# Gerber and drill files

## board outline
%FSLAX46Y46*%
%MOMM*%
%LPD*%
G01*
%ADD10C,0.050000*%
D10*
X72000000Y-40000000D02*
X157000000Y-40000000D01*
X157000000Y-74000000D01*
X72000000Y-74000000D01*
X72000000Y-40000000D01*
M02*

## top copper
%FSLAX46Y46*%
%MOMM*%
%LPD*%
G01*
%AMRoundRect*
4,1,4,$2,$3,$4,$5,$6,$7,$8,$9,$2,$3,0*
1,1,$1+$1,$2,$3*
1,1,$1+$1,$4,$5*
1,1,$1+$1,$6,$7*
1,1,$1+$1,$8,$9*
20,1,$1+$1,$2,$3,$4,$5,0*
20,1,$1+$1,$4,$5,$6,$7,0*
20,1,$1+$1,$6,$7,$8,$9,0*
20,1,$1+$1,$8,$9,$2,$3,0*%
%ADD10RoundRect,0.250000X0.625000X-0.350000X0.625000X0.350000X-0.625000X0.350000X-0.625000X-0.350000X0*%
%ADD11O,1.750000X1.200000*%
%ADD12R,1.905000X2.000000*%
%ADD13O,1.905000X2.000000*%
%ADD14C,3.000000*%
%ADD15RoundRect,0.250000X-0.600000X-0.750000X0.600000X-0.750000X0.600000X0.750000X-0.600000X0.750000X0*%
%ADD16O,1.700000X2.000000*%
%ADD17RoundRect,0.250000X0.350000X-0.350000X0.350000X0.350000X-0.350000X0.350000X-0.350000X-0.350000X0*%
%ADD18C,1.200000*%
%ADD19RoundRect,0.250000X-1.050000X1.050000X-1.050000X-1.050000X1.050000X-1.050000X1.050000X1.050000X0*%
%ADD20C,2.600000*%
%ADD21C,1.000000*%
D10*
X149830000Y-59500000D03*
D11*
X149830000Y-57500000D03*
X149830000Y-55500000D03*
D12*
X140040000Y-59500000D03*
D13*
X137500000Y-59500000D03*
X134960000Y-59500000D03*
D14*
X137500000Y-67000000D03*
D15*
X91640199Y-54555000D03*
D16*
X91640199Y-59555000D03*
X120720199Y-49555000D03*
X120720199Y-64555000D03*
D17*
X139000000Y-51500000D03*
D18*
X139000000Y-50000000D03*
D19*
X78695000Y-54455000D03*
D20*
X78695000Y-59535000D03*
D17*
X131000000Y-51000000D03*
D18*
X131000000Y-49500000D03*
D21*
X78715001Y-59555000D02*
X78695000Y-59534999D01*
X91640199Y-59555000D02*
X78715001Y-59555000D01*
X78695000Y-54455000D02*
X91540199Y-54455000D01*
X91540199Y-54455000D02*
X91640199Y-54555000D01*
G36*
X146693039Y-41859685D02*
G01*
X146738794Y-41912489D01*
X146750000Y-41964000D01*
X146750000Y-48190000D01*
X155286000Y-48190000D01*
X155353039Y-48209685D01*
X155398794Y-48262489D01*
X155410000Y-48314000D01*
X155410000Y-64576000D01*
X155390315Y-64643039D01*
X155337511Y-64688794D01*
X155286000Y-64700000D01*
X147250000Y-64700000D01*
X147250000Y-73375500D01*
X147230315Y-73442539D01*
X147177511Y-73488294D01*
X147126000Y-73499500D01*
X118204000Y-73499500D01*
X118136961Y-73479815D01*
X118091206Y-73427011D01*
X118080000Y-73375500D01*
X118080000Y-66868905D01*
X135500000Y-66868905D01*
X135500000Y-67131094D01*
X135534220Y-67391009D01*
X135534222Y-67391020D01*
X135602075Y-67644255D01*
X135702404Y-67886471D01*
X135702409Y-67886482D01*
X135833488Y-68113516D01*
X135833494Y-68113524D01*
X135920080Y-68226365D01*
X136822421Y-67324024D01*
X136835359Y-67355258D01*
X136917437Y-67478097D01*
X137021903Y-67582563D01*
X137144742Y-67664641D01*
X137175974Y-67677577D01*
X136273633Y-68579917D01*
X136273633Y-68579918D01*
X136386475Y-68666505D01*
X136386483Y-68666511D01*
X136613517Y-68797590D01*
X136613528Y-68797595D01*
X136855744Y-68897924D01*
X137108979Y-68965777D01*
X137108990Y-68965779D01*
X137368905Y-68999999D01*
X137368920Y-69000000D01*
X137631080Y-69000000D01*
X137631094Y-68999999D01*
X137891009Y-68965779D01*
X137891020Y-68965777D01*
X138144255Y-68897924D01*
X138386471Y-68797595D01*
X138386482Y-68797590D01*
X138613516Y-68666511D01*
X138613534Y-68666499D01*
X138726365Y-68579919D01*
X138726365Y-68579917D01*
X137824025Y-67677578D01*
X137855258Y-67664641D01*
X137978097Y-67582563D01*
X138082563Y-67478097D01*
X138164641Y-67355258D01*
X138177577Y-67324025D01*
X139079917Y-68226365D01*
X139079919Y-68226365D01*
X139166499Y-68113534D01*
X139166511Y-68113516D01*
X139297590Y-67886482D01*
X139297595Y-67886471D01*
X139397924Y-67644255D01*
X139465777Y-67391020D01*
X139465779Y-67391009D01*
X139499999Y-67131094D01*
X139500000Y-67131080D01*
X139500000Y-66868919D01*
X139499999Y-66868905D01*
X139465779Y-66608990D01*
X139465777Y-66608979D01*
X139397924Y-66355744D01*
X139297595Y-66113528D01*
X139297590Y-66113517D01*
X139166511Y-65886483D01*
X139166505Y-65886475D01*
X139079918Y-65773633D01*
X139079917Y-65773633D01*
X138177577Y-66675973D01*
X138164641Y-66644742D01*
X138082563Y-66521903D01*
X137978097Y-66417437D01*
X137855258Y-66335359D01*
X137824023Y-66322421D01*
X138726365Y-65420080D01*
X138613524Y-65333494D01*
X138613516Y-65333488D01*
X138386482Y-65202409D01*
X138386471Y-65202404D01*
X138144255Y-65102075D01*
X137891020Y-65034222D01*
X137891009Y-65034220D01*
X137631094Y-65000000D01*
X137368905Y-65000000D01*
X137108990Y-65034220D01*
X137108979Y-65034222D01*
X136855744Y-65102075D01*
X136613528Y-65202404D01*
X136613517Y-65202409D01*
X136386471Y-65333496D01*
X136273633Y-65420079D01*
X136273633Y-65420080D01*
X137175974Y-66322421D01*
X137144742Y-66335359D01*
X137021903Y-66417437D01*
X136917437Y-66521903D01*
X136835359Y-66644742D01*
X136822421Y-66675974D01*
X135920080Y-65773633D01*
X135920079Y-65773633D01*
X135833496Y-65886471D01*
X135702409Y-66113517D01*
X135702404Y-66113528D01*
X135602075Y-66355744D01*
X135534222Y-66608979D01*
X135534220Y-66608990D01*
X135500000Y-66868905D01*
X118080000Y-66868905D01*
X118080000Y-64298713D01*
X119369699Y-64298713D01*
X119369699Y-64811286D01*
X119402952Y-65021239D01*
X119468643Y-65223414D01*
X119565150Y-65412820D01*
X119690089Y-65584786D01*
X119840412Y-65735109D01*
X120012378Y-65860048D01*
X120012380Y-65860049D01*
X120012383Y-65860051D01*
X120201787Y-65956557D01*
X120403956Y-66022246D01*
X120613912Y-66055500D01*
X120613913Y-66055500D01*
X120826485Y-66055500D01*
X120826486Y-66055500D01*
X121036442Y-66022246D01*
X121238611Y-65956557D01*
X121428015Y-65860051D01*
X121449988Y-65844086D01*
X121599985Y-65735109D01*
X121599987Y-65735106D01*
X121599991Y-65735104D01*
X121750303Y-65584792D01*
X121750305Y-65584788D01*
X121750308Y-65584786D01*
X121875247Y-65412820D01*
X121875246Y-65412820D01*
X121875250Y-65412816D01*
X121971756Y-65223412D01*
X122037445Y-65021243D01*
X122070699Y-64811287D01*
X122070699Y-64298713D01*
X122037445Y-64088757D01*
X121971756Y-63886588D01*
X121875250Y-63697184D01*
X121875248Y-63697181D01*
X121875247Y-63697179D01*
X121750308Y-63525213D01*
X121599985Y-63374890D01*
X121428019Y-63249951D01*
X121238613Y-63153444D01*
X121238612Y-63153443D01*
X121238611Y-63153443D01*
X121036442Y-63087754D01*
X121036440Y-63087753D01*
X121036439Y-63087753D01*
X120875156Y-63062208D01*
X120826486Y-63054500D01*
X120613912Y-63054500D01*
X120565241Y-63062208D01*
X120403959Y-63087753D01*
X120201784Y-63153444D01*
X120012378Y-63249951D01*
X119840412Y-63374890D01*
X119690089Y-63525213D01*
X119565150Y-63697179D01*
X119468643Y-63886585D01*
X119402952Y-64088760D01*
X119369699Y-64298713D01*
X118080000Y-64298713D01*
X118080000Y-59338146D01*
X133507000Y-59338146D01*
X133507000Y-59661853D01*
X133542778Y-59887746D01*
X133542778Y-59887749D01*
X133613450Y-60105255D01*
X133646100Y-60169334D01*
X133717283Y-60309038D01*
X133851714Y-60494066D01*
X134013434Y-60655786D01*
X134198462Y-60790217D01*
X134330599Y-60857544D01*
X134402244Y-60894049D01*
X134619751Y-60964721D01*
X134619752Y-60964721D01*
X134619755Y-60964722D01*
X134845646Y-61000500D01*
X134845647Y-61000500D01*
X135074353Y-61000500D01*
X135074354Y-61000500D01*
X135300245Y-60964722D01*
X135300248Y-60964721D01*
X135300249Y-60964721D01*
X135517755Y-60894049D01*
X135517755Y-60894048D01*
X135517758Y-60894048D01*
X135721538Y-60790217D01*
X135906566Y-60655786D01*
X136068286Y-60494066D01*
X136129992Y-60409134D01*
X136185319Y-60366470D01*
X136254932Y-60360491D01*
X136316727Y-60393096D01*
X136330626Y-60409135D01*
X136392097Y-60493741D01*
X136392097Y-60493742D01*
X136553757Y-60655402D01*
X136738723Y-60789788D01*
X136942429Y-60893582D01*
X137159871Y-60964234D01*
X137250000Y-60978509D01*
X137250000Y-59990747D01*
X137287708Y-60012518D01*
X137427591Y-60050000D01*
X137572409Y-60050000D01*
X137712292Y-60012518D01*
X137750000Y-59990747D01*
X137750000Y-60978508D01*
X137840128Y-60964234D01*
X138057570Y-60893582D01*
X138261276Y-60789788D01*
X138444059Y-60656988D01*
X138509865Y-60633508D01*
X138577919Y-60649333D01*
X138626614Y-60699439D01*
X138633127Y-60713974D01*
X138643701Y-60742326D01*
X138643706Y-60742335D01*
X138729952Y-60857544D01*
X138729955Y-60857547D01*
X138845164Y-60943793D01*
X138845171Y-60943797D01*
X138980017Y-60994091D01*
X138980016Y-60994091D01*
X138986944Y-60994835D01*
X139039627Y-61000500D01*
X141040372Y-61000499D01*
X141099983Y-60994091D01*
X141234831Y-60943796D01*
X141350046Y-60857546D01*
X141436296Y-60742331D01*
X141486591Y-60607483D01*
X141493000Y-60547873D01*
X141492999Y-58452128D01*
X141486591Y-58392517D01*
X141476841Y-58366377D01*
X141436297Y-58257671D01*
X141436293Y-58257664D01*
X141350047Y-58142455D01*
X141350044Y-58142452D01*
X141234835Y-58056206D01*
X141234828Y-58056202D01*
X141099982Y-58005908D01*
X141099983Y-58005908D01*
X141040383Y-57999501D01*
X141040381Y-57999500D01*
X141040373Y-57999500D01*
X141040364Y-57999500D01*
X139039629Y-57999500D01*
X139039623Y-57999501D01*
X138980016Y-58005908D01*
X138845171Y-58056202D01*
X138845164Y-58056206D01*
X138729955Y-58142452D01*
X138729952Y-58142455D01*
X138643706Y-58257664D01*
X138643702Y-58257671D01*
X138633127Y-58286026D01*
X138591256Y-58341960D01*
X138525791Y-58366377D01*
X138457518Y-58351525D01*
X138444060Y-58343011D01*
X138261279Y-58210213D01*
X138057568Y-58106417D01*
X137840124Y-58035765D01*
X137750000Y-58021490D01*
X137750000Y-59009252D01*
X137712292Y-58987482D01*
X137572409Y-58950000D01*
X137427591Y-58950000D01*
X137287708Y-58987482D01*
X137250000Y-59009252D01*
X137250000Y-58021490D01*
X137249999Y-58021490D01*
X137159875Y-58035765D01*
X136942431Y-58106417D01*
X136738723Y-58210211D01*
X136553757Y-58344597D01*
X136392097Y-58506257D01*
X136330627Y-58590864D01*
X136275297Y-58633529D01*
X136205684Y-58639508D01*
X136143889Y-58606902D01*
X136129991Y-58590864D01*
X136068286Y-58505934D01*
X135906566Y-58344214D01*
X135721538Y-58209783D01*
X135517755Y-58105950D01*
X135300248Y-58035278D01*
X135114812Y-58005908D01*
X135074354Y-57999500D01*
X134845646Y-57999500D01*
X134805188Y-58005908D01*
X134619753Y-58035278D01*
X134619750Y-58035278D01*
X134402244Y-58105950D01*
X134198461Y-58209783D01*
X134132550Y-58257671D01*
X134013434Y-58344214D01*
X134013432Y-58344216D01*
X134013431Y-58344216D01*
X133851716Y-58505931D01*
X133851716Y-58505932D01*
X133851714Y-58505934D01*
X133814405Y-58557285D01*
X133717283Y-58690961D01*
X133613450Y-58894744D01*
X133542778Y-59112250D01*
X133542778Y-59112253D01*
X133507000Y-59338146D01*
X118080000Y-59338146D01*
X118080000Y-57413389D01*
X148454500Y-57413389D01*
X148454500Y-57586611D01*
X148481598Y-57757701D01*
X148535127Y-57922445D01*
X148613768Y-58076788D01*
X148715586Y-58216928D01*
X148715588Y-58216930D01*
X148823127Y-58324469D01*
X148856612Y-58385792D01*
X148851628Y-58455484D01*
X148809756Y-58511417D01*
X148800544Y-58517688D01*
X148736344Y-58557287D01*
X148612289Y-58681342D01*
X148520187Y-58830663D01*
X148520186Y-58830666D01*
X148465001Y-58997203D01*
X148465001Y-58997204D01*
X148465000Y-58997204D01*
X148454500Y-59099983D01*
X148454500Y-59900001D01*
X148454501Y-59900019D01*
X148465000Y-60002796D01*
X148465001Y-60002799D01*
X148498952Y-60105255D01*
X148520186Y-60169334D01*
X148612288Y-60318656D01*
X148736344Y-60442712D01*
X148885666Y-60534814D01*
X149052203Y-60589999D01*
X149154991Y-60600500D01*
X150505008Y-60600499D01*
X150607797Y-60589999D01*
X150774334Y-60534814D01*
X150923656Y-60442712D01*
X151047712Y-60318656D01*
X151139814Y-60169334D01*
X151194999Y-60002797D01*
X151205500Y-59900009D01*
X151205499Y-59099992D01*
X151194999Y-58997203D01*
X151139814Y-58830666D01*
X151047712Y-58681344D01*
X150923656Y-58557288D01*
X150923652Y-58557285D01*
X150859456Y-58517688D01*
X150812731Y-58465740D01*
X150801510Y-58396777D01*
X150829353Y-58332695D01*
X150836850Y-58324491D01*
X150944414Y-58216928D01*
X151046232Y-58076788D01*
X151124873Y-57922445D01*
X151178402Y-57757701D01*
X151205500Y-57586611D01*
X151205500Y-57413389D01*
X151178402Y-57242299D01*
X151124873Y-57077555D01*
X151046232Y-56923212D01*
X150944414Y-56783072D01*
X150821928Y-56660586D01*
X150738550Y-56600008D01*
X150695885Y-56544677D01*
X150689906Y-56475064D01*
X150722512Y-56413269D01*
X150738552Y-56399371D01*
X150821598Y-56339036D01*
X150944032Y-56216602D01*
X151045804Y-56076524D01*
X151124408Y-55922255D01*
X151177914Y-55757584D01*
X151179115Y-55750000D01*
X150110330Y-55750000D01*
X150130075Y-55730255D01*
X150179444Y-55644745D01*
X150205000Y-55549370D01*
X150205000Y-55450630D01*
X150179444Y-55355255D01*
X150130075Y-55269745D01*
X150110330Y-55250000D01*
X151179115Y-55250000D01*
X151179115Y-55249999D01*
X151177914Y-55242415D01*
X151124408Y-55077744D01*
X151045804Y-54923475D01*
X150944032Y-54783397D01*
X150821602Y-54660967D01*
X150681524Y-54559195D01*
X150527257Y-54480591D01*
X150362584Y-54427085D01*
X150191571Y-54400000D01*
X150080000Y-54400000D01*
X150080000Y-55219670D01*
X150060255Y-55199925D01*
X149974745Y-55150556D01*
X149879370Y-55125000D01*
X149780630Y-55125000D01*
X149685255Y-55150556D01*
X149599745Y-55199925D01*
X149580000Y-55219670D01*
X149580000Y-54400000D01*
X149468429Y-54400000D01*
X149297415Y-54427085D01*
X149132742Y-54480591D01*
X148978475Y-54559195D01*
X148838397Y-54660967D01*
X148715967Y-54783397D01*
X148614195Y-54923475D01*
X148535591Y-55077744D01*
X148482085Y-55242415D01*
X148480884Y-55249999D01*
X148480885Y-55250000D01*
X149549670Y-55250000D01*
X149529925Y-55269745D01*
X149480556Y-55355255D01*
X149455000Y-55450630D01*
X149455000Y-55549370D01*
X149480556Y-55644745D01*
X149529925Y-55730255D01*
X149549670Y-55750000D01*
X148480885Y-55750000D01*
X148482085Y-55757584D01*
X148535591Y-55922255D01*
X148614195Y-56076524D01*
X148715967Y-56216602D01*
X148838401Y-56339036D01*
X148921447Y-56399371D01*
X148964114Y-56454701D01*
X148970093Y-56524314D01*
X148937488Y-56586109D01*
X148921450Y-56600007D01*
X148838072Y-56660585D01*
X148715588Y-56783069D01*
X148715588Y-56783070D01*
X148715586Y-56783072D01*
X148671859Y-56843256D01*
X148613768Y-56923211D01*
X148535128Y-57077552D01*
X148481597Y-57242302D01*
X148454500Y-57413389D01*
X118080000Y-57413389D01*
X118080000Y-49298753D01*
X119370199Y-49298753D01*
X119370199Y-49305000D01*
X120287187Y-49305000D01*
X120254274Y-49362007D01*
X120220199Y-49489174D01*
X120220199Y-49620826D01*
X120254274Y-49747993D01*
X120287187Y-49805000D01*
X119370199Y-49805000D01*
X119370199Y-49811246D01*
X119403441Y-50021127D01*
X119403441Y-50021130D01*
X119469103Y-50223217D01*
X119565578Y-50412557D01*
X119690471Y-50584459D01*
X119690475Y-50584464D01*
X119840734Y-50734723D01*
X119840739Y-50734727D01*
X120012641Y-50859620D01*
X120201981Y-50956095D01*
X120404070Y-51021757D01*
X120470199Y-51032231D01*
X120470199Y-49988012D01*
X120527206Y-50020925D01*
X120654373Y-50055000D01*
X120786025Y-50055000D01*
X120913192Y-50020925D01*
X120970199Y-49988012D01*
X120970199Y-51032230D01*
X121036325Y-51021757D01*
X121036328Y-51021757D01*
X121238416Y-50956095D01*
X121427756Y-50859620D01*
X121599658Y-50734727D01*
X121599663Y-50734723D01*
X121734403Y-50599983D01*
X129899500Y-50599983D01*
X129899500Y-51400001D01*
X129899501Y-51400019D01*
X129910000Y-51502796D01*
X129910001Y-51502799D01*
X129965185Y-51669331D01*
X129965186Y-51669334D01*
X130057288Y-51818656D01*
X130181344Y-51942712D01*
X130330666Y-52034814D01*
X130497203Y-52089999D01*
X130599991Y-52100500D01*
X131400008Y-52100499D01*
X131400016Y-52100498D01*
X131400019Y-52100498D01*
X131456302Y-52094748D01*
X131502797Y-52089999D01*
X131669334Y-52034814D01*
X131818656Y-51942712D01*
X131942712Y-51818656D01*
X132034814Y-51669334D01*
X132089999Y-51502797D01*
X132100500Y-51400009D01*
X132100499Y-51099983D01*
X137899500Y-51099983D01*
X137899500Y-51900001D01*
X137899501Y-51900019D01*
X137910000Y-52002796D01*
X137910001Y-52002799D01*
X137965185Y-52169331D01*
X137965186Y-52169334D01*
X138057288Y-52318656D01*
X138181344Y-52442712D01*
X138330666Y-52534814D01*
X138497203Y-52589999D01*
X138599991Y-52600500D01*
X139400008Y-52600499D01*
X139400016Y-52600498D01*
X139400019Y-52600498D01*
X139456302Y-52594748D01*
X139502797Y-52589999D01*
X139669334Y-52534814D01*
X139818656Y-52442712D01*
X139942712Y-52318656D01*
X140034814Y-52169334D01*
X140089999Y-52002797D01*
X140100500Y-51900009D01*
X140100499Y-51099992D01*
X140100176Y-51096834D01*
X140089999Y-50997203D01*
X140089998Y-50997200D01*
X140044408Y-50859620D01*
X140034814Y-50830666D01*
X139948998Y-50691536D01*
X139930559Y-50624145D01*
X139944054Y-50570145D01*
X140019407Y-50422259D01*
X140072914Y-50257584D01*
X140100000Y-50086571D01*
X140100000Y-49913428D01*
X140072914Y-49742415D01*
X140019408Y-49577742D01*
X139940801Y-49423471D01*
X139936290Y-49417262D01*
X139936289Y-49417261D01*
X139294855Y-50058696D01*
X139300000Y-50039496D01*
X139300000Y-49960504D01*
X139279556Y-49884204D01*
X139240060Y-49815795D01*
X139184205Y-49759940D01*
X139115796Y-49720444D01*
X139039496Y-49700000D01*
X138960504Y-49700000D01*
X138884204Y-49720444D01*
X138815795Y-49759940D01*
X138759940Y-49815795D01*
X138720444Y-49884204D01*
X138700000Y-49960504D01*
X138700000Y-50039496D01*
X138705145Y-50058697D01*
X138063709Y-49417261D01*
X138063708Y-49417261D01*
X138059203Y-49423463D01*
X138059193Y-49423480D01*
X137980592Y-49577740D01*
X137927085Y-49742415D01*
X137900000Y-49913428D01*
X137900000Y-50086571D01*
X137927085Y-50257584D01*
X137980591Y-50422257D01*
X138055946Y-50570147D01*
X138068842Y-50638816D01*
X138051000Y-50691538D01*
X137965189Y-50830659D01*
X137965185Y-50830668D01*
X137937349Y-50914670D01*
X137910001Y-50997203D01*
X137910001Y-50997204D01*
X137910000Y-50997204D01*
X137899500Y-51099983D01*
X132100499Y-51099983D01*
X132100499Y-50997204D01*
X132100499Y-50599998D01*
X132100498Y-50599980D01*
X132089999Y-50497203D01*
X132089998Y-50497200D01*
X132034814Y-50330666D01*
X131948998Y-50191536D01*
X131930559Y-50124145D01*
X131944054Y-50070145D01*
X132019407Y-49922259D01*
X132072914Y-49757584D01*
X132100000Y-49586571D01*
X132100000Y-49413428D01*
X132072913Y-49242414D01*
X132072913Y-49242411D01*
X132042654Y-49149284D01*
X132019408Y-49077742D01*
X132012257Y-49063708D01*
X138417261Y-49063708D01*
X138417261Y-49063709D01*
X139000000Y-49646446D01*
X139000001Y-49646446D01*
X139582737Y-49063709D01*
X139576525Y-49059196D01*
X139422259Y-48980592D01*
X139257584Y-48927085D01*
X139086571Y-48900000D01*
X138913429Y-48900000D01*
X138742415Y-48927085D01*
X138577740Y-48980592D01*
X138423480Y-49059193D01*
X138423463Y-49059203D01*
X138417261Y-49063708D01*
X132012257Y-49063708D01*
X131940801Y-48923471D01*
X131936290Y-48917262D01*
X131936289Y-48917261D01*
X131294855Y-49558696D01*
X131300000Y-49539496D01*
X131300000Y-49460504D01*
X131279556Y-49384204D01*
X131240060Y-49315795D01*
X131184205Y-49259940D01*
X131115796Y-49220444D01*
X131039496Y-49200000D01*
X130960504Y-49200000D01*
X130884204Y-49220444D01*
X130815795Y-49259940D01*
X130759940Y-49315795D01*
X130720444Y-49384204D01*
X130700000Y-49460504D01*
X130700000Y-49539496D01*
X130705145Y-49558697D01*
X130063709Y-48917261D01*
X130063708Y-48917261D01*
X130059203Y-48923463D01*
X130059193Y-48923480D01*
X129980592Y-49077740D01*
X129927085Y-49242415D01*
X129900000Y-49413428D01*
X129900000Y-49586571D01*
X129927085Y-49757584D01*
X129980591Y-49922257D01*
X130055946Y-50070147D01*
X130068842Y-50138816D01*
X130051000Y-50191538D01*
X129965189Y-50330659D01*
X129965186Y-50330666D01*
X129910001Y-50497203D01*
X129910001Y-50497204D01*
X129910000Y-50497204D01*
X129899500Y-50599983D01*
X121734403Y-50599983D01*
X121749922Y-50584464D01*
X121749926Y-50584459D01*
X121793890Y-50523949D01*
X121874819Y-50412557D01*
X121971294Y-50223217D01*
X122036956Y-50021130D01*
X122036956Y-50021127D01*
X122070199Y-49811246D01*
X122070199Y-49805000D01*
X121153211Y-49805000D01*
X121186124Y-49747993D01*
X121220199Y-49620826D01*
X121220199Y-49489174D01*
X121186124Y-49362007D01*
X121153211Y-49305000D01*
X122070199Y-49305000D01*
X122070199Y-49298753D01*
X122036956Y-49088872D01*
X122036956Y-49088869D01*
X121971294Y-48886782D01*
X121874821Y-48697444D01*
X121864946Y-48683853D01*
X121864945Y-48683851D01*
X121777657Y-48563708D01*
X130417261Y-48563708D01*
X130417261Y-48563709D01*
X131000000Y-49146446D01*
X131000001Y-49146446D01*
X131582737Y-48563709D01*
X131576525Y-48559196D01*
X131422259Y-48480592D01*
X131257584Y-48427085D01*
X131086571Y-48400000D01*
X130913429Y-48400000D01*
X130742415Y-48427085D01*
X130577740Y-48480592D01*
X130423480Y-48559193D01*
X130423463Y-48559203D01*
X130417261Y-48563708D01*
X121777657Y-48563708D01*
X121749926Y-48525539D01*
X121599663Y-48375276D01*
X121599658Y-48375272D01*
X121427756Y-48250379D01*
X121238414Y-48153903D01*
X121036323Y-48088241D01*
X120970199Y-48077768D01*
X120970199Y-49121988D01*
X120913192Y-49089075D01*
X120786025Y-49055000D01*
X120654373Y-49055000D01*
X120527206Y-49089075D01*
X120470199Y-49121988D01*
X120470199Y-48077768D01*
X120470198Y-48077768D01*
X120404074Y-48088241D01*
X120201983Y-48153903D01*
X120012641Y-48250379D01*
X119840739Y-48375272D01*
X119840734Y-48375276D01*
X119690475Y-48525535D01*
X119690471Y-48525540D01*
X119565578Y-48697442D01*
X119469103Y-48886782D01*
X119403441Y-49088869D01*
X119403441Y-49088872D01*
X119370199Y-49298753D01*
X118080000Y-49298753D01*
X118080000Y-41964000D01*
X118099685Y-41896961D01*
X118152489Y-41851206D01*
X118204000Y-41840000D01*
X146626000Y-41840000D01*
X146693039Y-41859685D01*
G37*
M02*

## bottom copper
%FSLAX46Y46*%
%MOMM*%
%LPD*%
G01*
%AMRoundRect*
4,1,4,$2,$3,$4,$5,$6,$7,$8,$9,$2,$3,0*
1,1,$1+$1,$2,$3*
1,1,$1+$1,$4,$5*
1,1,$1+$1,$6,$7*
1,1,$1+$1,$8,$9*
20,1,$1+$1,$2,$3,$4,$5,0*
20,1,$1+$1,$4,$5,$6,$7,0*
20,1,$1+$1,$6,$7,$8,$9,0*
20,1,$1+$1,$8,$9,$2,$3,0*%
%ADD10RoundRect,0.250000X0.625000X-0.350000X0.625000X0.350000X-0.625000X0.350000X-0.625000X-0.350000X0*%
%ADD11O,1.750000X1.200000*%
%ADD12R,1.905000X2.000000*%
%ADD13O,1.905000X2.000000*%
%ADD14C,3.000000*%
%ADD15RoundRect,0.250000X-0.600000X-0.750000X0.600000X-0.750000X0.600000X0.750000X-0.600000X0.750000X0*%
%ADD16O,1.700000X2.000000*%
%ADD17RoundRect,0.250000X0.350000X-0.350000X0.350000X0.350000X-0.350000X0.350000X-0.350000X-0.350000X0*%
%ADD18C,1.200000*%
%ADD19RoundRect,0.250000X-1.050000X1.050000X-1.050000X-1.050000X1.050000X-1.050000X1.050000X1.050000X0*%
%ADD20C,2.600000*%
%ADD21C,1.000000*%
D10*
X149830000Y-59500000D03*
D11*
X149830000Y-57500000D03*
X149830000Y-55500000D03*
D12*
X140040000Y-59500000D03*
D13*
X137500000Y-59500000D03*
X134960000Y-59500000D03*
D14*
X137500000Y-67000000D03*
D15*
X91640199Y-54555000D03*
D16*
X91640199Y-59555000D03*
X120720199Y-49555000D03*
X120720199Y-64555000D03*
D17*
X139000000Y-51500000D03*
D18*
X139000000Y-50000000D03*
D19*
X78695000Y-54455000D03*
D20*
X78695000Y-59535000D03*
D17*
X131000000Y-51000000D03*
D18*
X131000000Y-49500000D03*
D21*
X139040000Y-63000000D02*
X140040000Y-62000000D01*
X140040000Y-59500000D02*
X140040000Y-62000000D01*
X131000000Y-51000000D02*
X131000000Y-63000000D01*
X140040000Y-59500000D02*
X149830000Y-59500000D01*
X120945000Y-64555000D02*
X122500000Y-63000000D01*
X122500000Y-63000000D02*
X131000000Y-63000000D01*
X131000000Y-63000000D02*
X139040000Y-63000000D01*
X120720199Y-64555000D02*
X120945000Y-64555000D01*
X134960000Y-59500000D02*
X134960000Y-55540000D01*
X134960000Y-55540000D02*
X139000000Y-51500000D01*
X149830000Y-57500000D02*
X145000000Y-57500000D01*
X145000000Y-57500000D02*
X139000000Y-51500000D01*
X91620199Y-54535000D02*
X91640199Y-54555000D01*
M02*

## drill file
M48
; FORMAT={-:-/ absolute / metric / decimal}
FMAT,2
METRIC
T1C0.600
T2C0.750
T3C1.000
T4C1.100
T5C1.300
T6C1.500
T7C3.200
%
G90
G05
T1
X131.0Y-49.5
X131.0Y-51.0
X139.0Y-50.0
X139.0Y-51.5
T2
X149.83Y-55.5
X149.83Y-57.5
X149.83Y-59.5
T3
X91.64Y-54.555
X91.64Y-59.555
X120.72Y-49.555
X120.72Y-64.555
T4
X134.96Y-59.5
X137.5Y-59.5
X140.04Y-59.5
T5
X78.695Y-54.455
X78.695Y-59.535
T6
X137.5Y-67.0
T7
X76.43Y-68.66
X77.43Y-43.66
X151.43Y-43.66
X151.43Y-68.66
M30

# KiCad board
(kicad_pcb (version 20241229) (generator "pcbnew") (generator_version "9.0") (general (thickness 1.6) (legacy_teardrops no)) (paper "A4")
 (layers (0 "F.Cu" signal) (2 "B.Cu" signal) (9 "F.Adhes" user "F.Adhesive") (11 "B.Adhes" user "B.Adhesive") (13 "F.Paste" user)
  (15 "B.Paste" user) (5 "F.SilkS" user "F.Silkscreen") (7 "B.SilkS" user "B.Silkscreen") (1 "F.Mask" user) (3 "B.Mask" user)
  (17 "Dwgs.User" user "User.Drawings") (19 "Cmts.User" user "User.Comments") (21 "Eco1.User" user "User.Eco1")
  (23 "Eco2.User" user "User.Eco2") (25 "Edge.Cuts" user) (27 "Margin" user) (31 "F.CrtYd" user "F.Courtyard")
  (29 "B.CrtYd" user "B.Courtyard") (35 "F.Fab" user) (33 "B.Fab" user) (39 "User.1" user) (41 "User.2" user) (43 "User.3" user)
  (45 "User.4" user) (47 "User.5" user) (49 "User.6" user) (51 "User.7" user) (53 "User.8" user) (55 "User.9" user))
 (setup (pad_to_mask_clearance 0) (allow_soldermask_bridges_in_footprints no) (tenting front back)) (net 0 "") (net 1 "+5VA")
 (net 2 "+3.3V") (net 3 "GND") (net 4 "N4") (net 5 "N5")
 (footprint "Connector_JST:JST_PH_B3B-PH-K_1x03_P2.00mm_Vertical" (layer "F.Cu") (at 149.83 59.5 90)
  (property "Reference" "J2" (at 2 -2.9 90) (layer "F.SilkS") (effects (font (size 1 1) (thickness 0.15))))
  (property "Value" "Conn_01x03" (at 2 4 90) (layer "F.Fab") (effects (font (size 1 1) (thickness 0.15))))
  (pad "1" thru_hole roundrect (at 0 0 90) (size 1.2 1.75) (drill 0.75) (layers "*.Cu" "*.Mask") (remove_unused_layers no)
   (roundrect_rratio 0.208333) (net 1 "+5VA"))
  (pad "2" thru_hole oval (at 2 0 90) (size 1.2 1.75) (drill 0.75) (layers "*.Cu" "*.Mask") (remove_unused_layers no) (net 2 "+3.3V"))
  (pad "3" thru_hole oval (at 4 0 90) (size 1.2 1.75) (drill 0.75) (layers "*.Cu" "*.Mask") (remove_unused_layers no) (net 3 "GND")))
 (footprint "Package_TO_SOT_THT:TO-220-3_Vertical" (layer "F.Cu") (at 140.04 59.5 180)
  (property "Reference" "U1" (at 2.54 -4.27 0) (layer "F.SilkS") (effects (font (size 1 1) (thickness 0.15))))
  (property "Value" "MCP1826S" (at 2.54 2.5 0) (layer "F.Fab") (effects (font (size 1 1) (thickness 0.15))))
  (pad "1" thru_hole rect (at 0 0 180) (size 1.905 2) (drill 1.1) (layers "*.Cu" "*.Mask") (remove_unused_layers no) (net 1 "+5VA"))
  (pad "2" thru_hole oval (at 2.54 0 180) (size 1.905 2) (drill 1.1) (layers "*.Cu" "*.Mask") (remove_unused_layers no) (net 3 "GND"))
  (pad "3" thru_hole oval (at 5.08 0 180) (size 1.905 2) (drill 1.1) (layers "*.Cu" "*.Mask") (remove_unused_layers no) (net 2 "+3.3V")))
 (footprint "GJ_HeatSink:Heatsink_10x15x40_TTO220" (layer "F.Cu") (at 137.5 67)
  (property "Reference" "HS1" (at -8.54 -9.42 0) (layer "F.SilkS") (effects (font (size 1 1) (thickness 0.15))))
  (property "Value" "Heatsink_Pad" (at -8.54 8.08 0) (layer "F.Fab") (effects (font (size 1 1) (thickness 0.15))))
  (pad "1" thru_hole circle (at 0 0) (size 3 3) (drill 1.5) (layers "*.Cu" "*.Mask") (remove_unused_layers no) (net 3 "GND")))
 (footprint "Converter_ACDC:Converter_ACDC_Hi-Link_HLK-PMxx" (layer "F.Cu") (at 91.640199 54.555)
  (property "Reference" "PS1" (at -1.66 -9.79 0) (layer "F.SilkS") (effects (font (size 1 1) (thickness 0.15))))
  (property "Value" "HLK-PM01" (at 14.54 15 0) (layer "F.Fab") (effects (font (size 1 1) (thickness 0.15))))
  (pad "1" thru_hole roundrect (at 0 0) (size 1.7 2) (drill 1) (layers "*.Cu" "*.Mask") (remove_unused_layers no)
   (roundrect_rratio 0.147059) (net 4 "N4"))
  (pad "2" thru_hole oval (at 0 5) (size 1.7 2) (drill 1) (layers "*.Cu" "*.Mask") (remove_unused_layers no) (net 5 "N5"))
  (pad "3" thru_hole oval (at 29.08 -5) (size 1.7 2) (drill 1) (layers "*.Cu" "*.Mask") (remove_unused_layers no) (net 3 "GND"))
  (pad "4" thru_hole oval (at 29.08 10) (size 1.7 2) (drill 1) (layers "*.Cu" "*.Mask") (remove_unused_layers no) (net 1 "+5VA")))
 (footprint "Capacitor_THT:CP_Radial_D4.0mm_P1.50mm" (layer "F.Cu") (at 139 51.5 90)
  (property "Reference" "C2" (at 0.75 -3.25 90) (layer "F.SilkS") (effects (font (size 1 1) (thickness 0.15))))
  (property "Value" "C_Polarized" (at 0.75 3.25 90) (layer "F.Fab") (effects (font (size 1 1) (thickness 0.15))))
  (pad "1" thru_hole roundrect (at 0 0 90) (size 1.2 1.2) (drill 0.6) (layers "*.Cu" "*.Mask") (remove_unused_layers no)
   (roundrect_rratio 0.208333) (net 2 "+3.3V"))
  (pad "2" thru_hole circle (at 1.5 0 90) (size 1.2 1.2) (drill 0.6) (layers "*.Cu" "*.Mask") (remove_unused_layers no) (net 3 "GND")))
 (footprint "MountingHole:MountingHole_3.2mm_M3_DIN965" (layer "F.Cu") (at 151.43 68.66)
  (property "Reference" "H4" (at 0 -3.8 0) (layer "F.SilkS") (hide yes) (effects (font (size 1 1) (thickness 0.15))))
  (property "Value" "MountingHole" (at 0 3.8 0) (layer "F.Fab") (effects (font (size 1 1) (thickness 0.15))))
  (pad "" np_thru_hole circle (at 0 0) (size 3.2 3.2) (drill 3.2) (layers "*.Cu" "*.Mask")))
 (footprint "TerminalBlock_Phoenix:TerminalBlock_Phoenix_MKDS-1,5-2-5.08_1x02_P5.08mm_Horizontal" (layer "F.Cu") (at 78.695 54.455 -90)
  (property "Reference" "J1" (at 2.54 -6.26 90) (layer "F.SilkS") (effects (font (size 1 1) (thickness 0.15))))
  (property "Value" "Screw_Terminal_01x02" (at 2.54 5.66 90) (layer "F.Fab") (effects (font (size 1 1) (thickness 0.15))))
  (pad "1" thru_hole roundrect (at 0 0 270) (size 2.6 2.6) (drill 1.3) (layers "*.Cu" "*.Mask") (remove_unused_layers no)
   (roundrect_rratio 0.096154) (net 4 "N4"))
  (pad "2" thru_hole circle (at 5.08 0 270) (size 2.6 2.6) (drill 1.3) (layers "*.Cu" "*.Mask") (remove_unused_layers no) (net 5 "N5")))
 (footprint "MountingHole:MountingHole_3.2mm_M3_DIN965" (layer "F.Cu") (at 77.43 43.66)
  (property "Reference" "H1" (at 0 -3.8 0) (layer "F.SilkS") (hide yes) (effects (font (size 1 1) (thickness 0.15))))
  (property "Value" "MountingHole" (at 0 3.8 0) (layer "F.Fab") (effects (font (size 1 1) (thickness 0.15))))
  (pad "" np_thru_hole circle (at 0 0) (size 3.2 3.2) (drill 3.2) (layers "*.Cu" "*.Mask")))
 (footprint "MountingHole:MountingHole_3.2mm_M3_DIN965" (layer "F.Cu") (at 151.43 43.66)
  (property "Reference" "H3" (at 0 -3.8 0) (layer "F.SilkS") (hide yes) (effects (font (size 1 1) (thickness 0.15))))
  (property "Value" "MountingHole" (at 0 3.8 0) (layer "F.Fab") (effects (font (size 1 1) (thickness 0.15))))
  (pad "" np_thru_hole circle (at 0 0) (size 3.2 3.2) (drill 3.2) (layers "*.Cu" "*.Mask")))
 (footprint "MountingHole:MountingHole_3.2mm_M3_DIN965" (layer "F.Cu") (at 76.43 68.66)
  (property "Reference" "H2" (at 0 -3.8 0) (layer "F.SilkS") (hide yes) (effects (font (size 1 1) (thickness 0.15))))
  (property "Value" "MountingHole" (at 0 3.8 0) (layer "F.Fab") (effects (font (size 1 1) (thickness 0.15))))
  (pad "" np_thru_hole circle (at 0 0) (size 3.2 3.2) (drill 3.2) (layers "*.Cu" "*.Mask")))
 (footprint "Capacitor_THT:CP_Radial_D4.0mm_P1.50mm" (layer "F.Cu") (at 131 51 90)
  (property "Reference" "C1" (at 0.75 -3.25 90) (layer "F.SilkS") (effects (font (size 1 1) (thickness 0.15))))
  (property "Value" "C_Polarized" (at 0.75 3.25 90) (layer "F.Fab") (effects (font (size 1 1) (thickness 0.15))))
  (pad "1" thru_hole roundrect (at 0 0 90) (size 1.2 1.2) (drill 0.6) (layers "*.Cu" "*.Mask") (remove_unused_layers no)
   (roundrect_rratio 0.208333) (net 1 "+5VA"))
  (pad "2" thru_hole circle (at 1.5 0 90) (size 1.2 1.2) (drill 0.6) (layers "*.Cu" "*.Mask") (remove_unused_layers no) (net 3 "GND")))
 (gr_rect (start 72 40) (end 157 74) (stroke (width 0.05) (type default)) (fill no) (layer "Edge.Cuts"))
 (segment (start 139.04 63) (end 140.04 62) (width 1) (layer "B.Cu") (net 1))
 (segment (start 140.04 59.5) (end 140.04 62) (width 1) (layer "B.Cu") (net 1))
 (segment (start 131 51) (end 131 63) (width 1) (layer "B.Cu") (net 1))
 (segment (start 140.04 59.5) (end 149.83 59.5) (width 1) (layer "B.Cu") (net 1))
 (segment (start 120.945 64.555) (end 122.5 63) (width 1) (layer "B.Cu") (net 1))
 (segment (start 122.5 63) (end 131 63) (width 1) (layer "B.Cu") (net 1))
 (segment (start 131 63) (end 139.04 63) (width 1) (layer "B.Cu") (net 1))
 (segment (start 120.720199 64.555) (end 120.945 64.555) (width 1) (layer "B.Cu") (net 1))
 (segment (start 134.96 59.5) (end 134.96 55.54) (width 1) (layer "B.Cu") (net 2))
 (segment (start 134.96 55.54) (end 139 51.5) (width 1) (layer "B.Cu") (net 2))
 (segment (start 149.83 57.5) (end 145 57.5) (width 1) (layer "B.Cu") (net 2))
 (segment (start 145 57.5) (end 139 51.5) (width 1) (layer "B.Cu") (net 2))
 (segment (start 78.715001 59.555) (end 78.695 59.534999) (width 1) (layer "F.Cu") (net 5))
 (segment (start 91.640199 59.555) (end 78.715001 59.555) (width 1) (layer "F.Cu") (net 5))
 (segment (start 78.695 54.455) (end 91.540199 54.455) (width 1) (layer "F.Cu") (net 4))
 (segment (start 91.540199 54.455) (end 91.640199 54.555) (width 1) (layer "F.Cu") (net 4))
 (segment (start 91.620199 54.535) (end 91.640199 54.555) (width 1) (layer "B.Cu") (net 4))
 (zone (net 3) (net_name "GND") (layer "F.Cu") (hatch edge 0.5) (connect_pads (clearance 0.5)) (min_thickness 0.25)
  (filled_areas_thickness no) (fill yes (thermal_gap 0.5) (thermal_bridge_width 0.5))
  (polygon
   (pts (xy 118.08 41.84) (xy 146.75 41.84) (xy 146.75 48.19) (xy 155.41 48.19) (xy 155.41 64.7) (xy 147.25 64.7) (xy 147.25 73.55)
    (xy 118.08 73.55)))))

